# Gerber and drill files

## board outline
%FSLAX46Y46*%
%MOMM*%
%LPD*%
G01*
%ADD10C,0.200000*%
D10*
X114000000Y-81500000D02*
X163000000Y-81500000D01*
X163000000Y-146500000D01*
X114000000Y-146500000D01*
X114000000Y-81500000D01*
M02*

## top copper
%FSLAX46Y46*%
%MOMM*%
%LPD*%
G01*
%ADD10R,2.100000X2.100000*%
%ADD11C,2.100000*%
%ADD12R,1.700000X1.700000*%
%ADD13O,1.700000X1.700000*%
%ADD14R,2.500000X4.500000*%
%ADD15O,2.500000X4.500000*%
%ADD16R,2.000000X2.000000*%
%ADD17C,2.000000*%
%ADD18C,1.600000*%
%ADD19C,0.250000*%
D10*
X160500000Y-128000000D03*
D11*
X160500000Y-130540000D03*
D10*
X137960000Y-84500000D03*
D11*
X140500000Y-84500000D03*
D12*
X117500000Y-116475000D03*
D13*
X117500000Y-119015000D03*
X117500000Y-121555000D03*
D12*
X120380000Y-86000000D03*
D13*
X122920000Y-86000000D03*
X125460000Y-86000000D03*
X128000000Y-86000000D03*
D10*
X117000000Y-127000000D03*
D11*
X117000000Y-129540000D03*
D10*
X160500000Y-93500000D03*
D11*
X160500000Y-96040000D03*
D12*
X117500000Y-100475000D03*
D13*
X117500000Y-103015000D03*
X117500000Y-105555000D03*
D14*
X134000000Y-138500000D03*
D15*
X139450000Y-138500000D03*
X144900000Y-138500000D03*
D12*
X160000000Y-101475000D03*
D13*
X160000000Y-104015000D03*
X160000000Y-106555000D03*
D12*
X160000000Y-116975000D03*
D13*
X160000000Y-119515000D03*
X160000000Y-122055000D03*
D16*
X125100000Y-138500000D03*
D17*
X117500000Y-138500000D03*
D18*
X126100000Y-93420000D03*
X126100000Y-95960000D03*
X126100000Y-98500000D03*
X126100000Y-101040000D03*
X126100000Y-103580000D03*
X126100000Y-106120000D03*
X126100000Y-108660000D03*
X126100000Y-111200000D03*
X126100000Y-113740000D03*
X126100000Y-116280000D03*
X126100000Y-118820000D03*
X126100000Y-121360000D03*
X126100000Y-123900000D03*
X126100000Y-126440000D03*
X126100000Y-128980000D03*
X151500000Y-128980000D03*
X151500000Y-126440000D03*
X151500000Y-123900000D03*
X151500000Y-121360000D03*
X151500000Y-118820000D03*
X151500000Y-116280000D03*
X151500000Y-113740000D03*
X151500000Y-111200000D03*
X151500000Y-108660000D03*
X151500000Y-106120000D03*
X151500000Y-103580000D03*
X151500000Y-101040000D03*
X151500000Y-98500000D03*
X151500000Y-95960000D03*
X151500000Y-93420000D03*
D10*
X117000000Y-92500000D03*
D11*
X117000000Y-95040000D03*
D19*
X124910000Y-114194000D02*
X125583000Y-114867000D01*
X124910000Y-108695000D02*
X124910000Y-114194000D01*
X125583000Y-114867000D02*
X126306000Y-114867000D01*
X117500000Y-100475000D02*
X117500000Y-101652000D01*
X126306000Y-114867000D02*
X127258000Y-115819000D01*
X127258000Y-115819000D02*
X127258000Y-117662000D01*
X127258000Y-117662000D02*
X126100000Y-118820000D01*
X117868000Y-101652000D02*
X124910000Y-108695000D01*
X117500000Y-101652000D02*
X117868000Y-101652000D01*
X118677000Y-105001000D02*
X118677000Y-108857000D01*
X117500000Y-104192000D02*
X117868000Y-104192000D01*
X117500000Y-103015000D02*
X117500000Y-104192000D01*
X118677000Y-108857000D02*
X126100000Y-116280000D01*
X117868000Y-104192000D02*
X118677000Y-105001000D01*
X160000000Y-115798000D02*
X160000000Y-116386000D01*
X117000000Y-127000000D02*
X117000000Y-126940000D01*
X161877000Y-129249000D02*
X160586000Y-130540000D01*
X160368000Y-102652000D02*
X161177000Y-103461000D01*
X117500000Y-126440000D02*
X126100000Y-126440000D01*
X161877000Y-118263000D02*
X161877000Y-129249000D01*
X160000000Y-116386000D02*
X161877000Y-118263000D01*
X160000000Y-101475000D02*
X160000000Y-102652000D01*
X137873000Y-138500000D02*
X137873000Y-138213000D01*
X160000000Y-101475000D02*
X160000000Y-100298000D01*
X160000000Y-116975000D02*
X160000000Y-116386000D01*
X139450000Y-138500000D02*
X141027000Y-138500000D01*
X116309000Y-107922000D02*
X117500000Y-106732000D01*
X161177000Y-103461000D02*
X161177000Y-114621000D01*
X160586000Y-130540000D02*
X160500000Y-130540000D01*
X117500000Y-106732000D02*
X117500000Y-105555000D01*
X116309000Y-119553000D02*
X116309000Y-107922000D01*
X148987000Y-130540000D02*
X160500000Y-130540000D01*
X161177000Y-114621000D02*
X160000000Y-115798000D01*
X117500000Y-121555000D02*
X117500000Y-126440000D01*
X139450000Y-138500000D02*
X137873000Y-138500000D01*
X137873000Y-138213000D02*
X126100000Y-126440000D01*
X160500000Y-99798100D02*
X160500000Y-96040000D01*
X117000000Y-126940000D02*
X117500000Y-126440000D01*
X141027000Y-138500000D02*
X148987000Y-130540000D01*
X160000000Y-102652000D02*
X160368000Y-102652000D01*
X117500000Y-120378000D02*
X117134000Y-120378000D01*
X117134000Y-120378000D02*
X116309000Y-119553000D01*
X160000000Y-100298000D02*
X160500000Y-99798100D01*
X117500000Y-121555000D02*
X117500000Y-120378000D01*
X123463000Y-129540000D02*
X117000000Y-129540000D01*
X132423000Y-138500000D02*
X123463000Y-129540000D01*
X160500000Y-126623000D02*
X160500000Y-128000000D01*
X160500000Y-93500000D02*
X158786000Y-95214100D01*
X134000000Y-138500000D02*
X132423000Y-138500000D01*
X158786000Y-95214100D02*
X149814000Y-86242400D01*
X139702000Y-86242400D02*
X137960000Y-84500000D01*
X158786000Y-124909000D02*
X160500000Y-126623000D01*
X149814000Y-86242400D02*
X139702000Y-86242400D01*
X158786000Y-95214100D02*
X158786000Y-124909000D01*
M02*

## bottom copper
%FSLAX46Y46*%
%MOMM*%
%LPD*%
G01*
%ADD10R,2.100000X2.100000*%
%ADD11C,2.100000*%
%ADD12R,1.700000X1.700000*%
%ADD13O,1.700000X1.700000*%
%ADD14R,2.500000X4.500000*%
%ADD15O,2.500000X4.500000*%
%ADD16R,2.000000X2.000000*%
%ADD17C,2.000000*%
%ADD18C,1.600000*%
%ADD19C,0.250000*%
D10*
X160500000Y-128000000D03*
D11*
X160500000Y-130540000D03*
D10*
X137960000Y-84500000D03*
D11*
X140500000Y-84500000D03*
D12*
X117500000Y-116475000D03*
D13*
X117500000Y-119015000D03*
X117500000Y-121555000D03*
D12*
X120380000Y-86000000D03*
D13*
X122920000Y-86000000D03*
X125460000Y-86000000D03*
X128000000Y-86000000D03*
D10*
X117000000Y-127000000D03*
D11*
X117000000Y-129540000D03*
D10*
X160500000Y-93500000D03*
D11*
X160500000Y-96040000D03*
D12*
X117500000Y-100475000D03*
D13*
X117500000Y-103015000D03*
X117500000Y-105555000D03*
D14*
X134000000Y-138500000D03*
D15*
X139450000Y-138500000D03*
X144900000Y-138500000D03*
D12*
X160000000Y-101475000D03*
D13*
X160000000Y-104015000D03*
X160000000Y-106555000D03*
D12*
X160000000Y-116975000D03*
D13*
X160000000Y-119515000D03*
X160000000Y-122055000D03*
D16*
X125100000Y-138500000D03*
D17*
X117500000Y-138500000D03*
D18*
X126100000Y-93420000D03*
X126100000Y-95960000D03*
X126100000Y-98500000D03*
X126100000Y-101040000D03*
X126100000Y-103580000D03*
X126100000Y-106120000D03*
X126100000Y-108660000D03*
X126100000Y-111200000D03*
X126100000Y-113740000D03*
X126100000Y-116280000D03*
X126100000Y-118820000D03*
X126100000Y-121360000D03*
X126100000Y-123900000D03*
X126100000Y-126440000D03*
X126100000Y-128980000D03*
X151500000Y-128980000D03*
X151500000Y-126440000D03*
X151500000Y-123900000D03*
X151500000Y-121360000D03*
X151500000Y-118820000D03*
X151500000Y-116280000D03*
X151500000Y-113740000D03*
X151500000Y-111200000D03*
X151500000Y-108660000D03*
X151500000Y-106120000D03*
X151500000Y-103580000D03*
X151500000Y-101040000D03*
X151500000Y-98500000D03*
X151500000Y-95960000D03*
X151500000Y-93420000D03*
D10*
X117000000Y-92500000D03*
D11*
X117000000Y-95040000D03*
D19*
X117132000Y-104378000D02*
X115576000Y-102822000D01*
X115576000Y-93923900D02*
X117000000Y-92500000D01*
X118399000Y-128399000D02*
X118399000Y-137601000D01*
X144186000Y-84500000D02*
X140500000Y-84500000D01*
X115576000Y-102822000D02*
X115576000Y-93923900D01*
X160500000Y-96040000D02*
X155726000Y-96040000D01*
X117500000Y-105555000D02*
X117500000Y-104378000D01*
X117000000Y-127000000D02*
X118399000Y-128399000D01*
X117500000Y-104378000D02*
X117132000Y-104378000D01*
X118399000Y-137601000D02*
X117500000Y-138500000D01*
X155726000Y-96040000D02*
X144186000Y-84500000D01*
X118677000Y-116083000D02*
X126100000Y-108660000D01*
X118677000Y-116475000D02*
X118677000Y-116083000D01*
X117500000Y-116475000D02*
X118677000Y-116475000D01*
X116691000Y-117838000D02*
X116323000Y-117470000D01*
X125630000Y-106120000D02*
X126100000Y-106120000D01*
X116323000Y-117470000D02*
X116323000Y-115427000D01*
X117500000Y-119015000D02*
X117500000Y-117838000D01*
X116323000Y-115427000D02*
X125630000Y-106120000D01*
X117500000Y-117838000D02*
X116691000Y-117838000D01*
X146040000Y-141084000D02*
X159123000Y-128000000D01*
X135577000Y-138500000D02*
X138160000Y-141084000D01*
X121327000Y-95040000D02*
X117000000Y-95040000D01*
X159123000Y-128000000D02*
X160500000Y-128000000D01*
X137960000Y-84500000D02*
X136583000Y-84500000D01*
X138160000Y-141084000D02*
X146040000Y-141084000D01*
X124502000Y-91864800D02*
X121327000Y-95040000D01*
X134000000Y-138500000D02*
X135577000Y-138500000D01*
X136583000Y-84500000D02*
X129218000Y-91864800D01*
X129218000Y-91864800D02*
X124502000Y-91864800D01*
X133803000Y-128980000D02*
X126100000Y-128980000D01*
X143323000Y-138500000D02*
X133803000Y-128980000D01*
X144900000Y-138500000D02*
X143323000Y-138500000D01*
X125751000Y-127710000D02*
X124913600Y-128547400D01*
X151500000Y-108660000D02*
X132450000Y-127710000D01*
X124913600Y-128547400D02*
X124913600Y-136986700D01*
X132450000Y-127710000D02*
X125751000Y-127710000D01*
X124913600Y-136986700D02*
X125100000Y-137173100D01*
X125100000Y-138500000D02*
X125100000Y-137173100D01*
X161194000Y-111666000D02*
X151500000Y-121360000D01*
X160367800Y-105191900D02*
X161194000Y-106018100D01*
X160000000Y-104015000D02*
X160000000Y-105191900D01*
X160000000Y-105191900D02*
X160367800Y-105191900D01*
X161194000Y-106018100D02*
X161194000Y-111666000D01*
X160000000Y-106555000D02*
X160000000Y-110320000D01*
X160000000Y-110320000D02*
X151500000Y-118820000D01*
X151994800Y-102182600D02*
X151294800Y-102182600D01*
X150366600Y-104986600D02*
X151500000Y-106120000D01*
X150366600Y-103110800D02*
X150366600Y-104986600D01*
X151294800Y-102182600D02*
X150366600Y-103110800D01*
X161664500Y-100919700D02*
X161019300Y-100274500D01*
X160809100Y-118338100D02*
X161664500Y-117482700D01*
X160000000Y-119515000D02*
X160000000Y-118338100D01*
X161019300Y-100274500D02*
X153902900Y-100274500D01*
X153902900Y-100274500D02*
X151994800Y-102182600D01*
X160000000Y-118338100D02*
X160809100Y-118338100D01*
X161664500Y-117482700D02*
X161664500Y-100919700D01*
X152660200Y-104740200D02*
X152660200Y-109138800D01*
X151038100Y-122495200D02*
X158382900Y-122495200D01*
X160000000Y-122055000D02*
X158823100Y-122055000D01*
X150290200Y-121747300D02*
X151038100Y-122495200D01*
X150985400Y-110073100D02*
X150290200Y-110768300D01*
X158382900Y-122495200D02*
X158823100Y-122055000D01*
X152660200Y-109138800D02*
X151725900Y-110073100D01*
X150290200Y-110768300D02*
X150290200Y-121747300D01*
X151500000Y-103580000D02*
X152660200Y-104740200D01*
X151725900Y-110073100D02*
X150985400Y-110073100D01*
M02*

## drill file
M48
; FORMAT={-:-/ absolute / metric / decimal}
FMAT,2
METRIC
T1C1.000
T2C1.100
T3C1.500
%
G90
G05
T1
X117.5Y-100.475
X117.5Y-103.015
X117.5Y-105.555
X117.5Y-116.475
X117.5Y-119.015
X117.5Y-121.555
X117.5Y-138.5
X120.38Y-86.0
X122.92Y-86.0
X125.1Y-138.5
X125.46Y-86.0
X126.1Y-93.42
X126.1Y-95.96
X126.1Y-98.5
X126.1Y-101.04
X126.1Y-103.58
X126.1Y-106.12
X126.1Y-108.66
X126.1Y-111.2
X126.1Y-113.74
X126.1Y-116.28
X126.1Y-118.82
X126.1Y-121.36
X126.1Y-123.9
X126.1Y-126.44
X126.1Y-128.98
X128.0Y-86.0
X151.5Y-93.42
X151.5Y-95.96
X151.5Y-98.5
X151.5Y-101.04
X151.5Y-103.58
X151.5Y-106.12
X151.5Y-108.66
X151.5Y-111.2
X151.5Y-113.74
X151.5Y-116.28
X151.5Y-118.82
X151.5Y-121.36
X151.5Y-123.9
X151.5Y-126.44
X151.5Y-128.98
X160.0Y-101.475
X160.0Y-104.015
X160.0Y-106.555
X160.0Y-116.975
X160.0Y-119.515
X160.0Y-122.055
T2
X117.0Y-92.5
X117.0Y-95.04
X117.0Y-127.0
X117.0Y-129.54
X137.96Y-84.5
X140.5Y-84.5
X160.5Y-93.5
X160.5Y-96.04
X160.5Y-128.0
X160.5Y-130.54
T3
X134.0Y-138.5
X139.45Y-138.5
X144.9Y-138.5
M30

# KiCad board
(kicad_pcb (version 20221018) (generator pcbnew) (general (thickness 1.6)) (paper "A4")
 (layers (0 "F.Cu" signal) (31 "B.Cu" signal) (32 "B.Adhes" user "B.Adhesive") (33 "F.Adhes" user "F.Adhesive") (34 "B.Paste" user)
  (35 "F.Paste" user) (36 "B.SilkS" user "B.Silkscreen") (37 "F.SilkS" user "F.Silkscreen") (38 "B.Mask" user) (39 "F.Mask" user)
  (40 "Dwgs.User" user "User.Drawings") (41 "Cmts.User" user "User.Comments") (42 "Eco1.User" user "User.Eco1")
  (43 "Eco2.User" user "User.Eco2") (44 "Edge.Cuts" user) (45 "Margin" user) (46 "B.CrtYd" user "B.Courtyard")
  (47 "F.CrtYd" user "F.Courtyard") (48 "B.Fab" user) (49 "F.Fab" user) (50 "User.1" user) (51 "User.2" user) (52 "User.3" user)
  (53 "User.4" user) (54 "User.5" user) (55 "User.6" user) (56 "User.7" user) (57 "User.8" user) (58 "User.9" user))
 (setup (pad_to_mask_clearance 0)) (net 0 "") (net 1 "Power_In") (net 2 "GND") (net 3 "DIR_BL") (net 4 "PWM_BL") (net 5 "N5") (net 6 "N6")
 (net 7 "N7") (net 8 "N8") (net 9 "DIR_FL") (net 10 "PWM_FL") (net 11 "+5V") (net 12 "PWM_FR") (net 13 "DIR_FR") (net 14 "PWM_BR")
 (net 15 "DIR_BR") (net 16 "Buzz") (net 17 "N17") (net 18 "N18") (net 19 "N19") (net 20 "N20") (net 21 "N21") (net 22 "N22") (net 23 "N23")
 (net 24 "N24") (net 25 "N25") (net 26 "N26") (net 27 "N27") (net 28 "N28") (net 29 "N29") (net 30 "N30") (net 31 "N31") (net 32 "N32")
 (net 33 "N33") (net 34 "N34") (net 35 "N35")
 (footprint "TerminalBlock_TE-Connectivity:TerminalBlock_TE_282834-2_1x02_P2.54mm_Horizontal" (layer "F.Cu") (at 160.5 128 -90)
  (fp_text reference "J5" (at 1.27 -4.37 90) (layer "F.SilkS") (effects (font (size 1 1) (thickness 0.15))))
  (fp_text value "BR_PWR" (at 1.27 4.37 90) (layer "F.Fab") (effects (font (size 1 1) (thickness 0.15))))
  (pad "1" thru_hole rect (at 0 0 270) (size 2.1 2.1) (drill 1.1) (layers "*.Cu" "*.Mask") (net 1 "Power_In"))
  (pad "2" thru_hole circle (at 2.54 0 270) (size 2.1 2.1) (drill 1.1) (layers "*.Cu" "*.Mask") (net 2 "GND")))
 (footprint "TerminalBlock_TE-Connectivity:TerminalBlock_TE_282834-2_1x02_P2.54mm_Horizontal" (layer "F.Cu") (at 137.96 84.5)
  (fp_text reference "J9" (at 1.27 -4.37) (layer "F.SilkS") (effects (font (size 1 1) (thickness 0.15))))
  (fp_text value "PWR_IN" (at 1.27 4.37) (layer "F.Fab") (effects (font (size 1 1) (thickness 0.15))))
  (pad "1" thru_hole rect (at 0 0) (size 2.1 2.1) (drill 1.1) (layers "*.Cu" "*.Mask") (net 1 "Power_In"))
  (pad "2" thru_hole circle (at 2.54 0) (size 2.1 2.1) (drill 1.1) (layers "*.Cu" "*.Mask") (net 2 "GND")))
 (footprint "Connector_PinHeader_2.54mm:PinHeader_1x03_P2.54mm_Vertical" (layer "F.Cu") (at 117.5 116.475)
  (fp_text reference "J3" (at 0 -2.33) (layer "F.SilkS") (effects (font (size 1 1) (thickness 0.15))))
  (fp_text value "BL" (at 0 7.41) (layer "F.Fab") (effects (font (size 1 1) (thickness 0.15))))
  (pad "1" thru_hole rect (at 0 0) (size 1.7 1.7) (drill 1) (layers "*.Cu" "*.Mask") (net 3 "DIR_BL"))
  (pad "2" thru_hole oval (at 0 2.54) (size 1.7 1.7) (drill 1) (layers "*.Cu" "*.Mask") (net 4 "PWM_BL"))
  (pad "3" thru_hole oval (at 0 5.08) (size 1.7 1.7) (drill 1) (layers "*.Cu" "*.Mask") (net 2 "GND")))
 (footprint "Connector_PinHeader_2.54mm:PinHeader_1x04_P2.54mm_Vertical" (layer "F.Cu") (at 120.38 86 90)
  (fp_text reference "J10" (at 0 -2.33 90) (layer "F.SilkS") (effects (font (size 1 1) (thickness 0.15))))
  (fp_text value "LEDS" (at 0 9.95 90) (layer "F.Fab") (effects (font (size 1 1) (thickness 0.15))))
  (pad "1" thru_hole rect (at 0 0 90) (size 1.7 1.7) (drill 1) (layers "*.Cu" "*.Mask") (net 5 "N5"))
  (pad "2" thru_hole oval (at 0 2.54 90) (size 1.7 1.7) (drill 1) (layers "*.Cu" "*.Mask") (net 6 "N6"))
  (pad "3" thru_hole oval (at 0 5.08 90) (size 1.7 1.7) (drill 1) (layers "*.Cu" "*.Mask") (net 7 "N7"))
  (pad "4" thru_hole oval (at 0 7.62 90) (size 1.7 1.7) (drill 1) (layers "*.Cu" "*.Mask") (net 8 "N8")))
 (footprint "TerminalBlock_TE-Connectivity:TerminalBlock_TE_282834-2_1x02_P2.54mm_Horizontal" (layer "F.Cu") (at 117 127 -90)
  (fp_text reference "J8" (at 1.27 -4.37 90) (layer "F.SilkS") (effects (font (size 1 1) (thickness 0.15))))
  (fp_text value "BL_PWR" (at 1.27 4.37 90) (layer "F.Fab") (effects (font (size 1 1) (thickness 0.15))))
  (pad "1" thru_hole rect (at 0 0 270) (size 2.1 2.1) (drill 1.1) (layers "*.Cu" "*.Mask") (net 2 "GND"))
  (pad "2" thru_hole circle (at 2.54 0 270) (size 2.1 2.1) (drill 1.1) (layers "*.Cu" "*.Mask") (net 1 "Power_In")))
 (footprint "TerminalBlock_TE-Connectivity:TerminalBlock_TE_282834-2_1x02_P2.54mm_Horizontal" (layer "F.Cu") (at 160.5 93.5 -90)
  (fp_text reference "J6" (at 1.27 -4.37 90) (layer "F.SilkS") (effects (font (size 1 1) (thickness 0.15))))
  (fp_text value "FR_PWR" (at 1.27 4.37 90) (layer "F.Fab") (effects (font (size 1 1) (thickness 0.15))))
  (pad "1" thru_hole rect (at 0 0 270) (size 2.1 2.1) (drill 1.1) (layers "*.Cu" "*.Mask") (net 1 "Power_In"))
  (pad "2" thru_hole circle (at 2.54 0 270) (size 2.1 2.1) (drill 1.1) (layers "*.Cu" "*.Mask") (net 2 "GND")))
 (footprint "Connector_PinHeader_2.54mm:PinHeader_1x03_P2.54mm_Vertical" (layer "F.Cu") (at 117.5 100.475)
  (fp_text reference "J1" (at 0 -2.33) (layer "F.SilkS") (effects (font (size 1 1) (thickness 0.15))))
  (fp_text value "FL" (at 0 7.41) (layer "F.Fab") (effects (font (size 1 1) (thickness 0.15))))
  (pad "1" thru_hole rect (at 0 0) (size 1.7 1.7) (drill 1) (layers "*.Cu" "*.Mask") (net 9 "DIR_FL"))
  (pad "2" thru_hole oval (at 0 2.54) (size 1.7 1.7) (drill 1) (layers "*.Cu" "*.Mask") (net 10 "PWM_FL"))
  (pad "3" thru_hole oval (at 0 5.08) (size 1.7 1.7) (drill 1) (layers "*.Cu" "*.Mask") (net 2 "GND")))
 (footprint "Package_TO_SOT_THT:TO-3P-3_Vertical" (layer "F.Cu") (at 134 138.5)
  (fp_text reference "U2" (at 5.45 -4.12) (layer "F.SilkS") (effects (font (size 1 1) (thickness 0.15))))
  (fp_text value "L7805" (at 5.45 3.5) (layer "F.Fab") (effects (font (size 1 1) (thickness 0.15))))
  (pad "1" thru_hole rect (at 0 0) (size 2.5 4.5) (drill 1.5) (layers "*.Cu" "*.Mask") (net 1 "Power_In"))
  (pad "2" thru_hole oval (at 5.45 0) (size 2.5 4.5) (drill 1.5) (layers "*.Cu" "*.Mask") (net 2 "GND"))
  (pad "3" thru_hole oval (at 10.9 0) (size 2.5 4.5) (drill 1.5) (layers "*.Cu" "*.Mask") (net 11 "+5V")))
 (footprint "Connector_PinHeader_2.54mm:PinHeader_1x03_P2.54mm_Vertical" (layer "F.Cu") (at 160 101.475)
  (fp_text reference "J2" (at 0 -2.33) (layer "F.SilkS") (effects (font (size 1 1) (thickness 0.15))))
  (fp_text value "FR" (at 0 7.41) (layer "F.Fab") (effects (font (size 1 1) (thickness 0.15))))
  (pad "1" thru_hole rect (at 0 0) (size 1.7 1.7) (drill 1) (layers "*.Cu" "*.Mask") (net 2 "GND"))
  (pad "2" thru_hole oval (at 0 2.54) (size 1.7 1.7) (drill 1) (layers "*.Cu" "*.Mask") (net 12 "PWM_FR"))
  (pad "3" thru_hole oval (at 0 5.08) (size 1.7 1.7) (drill 1) (layers "*.Cu" "*.Mask") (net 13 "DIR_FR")))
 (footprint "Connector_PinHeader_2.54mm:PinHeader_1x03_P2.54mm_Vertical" (layer "F.Cu") (at 160 116.975)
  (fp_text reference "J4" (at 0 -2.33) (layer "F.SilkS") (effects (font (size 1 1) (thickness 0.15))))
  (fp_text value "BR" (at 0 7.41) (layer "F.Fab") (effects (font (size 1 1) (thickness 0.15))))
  (pad "1" thru_hole rect (at 0 0) (size 1.7 1.7) (drill 1) (layers "*.Cu" "*.Mask") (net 2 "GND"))
  (pad "2" thru_hole oval (at 0 2.54) (size 1.7 1.7) (drill 1) (layers "*.Cu" "*.Mask") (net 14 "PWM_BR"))
  (pad "3" thru_hole oval (at 0 5.08) (size 1.7 1.7) (drill 1) (layers "*.Cu" "*.Mask") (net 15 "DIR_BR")))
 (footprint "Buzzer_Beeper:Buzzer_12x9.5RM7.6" (layer "F.Cu") (at 125.1 138.5 180)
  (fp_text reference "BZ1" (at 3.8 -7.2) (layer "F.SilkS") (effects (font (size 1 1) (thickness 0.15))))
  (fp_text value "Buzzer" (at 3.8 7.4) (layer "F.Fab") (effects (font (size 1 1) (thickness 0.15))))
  (pad "1" thru_hole rect (at 0 0 180) (size 2 2) (drill 1) (layers "*.Cu" "*.Mask") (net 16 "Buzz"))
  (pad "2" thru_hole circle (at 7.6 0 180) (size 2 2) (drill 1) (layers "*.Cu" "*.Mask") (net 2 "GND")))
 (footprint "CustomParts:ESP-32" (layer "F.Cu") (at 138.8 111.2)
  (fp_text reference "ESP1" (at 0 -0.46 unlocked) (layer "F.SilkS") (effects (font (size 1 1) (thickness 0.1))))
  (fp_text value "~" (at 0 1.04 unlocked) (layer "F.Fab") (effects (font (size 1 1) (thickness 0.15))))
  (pad "1" thru_hole circle (at -12.7 -17.78) (size 1.6 1.6) (drill 1) (layers "*.Cu" "*.Mask") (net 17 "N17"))
  (pad "2" thru_hole circle (at -12.7 -15.24) (size 1.6 1.6) (drill 1) (layers "*.Cu" "*.Mask") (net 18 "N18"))
  (pad "3" thru_hole circle (at -12.7 -12.7) (size 1.6 1.6) (drill 1) (layers "*.Cu" "*.Mask") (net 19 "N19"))
  (pad "4" thru_hole circle (at -12.7 -10.16) (size 1.6 1.6) (drill 1) (layers "*.Cu" "*.Mask") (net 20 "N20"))
  (pad "5" thru_hole circle (at -12.7 -7.62) (size 1.6 1.6) (drill 1) (layers "*.Cu" "*.Mask") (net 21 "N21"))
  (pad "6" thru_hole circle (at -12.7 -5.08) (size 1.6 1.6) (drill 1) (layers "*.Cu" "*.Mask") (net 4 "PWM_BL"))
  (pad "7" thru_hole circle (at -12.7 -2.54) (size 1.6 1.6) (drill 1) (layers "*.Cu" "*.Mask") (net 3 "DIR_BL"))
  (pad "8" thru_hole circle (at -12.7 0) (size 1.6 1.6) (drill 1) (layers "*.Cu" "*.Mask") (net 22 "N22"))
  (pad "9" thru_hole circle (at -12.7 2.54) (size 1.6 1.6) (drill 1) (layers "*.Cu" "*.Mask") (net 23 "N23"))
  (pad "10" thru_hole circle (at -12.7 5.08) (size 1.6 1.6) (drill 1) (layers "*.Cu" "*.Mask") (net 10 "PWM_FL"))
  (pad "11" thru_hole circle (at -12.7 7.62) (size 1.6 1.6) (drill 1) (layers "*.Cu" "*.Mask") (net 9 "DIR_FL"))
  (pad "12" thru_hole circle (at -12.7 10.16) (size 1.6 1.6) (drill 1) (layers "*.Cu" "*.Mask") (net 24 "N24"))
  (pad "13" thru_hole circle (at -12.7 12.7) (size 1.6 1.6) (drill 1) (layers "*.Cu" "*.Mask") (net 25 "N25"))
  (pad "14" thru_hole circle (at -12.7 15.24) (size 1.6 1.6) (drill 1) (layers "*.Cu" "*.Mask") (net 2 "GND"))
  (pad "15" thru_hole circle (at -12.7 17.78) (size 1.6 1.6) (drill 1) (layers "*.Cu" "*.Mask") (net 11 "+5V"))
  (pad "16" thru_hole circle (at 12.7 17.78) (size 1.6 1.6) (drill 1) (layers "*.Cu" "*.Mask") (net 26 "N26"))
  (pad "17" thru_hole circle (at 12.7 15.24) (size 1.6 1.6) (drill 1) (layers "*.Cu" "*.Mask") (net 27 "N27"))
  (pad "18" thru_hole circle (at 12.7 12.7) (size 1.6 1.6) (drill 1) (layers "*.Cu" "*.Mask") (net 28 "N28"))
  (pad "19" thru_hole circle (at 12.7 10.16) (size 1.6 1.6) (drill 1) (layers "*.Cu" "*.Mask") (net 12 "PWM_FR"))
  (pad "20" thru_hole circle (at 12.7 7.62) (size 1.6 1.6) (drill 1) (layers "*.Cu" "*.Mask") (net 13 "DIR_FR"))
  (pad "21" thru_hole circle (at 12.7 5.08) (size 1.6 1.6) (drill 1) (layers "*.Cu" "*.Mask") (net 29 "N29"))
  (pad "22" thru_hole circle (at 12.7 2.54) (size 1.6 1.6) (drill 1) (layers "*.Cu" "*.Mask") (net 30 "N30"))
  (pad "23" thru_hole circle (at 12.7 0) (size 1.6 1.6) (drill 1) (layers "*.Cu" "*.Mask") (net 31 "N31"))
  (pad "24" thru_hole circle (at 12.7 -2.54) (size 1.6 1.6) (drill 1) (layers "*.Cu" "*.Mask") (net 16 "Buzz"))
  (pad "25" thru_hole circle (at 12.7 -5.08) (size 1.6 1.6) (drill 1) (layers "*.Cu" "*.Mask") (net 14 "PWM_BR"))
  (pad "26" thru_hole circle (at 12.7 -7.62) (size 1.6 1.6) (drill 1) (layers "*.Cu" "*.Mask") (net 15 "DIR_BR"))
  (pad "27" thru_hole circle (at 12.7 -10.16) (size 1.6 1.6) (drill 1) (layers "*.Cu" "*.Mask") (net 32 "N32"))
  (pad "28" thru_hole circle (at 12.7 -12.7) (size 1.6 1.6) (drill 1) (layers "*.Cu" "*.Mask") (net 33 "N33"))
  (pad "29" thru_hole circle (at 12.7 -15.24) (size 1.6 1.6) (drill 1) (layers "*.Cu" "*.Mask") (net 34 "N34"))
  (pad "30" thru_hole circle (at 12.7 -17.78) (size 1.6 1.6) (drill 1) (layers "*.Cu" "*.Mask") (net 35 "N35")))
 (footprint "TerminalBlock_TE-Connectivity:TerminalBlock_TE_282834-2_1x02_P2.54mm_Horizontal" (layer "F.Cu") (at 117 92.5 -90)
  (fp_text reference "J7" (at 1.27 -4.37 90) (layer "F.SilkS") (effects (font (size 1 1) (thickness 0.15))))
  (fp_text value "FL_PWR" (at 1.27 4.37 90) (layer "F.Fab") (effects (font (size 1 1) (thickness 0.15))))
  (pad "1" thru_hole rect (at 0 0 270) (size 2.1 2.1) (drill 1.1) (layers "*.Cu" "*.Mask") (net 2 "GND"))
  (pad "2" thru_hole circle (at 2.54 0 270) (size 2.1 2.1) (drill 1.1) (layers "*.Cu" "*.Mask") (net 1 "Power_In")))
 (gr_rect (start 114 81.5) (end 163 146.5) (stroke (width 0.2) (type default)) (fill none) (layer "Edge.Cuts"))
 (segment (start 124.91 114.194) (end 125.583 114.867) (width 0.25) (layer "F.Cu") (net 9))
 (segment (start 124.91 108.695) (end 124.91 114.194) (width 0.25) (layer "F.Cu") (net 9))
 (segment (start 125.583 114.867) (end 126.306 114.867) (width 0.25) (layer "F.Cu") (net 9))
 (segment (start 117.5 100.475) (end 117.5 101.652) (width 0.25) (layer "F.Cu") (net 9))
 (segment (start 126.306 114.867) (end 127.258 115.819) (width 0.25) (layer "F.Cu") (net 9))
 (segment (start 127.258 115.819) (end 127.258 117.662) (width 0.25) (layer "F.Cu") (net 9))
 (segment (start 127.258 117.662) (end 126.1 118.82) (width 0.25) (layer "F.Cu") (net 9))
 (segment (start 117.868 101.652) (end 124.91 108.695) (width 0.25) (layer "F.Cu") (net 9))
 (segment (start 117.5 101.652) (end 117.868 101.652) (width 0.25) (layer "F.Cu") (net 9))
 (segment (start 118.677 105.001) (end 118.677 108.857) (width 0.25) (layer "F.Cu") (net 10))
 (segment (start 117.5 104.192) (end 117.868 104.192) (width 0.25) (layer "F.Cu") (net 10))
 (segment (start 117.5 103.015) (end 117.5 104.192) (width 0.25) (layer "F.Cu") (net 10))
 (segment (start 118.677 108.857) (end 126.1 116.28) (width 0.25) (layer "F.Cu") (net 10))
 (segment (start 117.868 104.192) (end 118.677 105.001) (width 0.25) (layer "F.Cu") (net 10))
 (segment (start 160 115.798) (end 160 116.386) (width 0.25) (layer "F.Cu") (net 2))
 (segment (start 117 127) (end 117 126.94) (width 0.25) (layer "F.Cu") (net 2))
 (segment (start 161.877 129.249) (end 160.586 130.54) (width 0.25) (layer "F.Cu") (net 2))
 (segment (start 160.368 102.652) (end 161.177 103.461) (width 0.25) (layer "F.Cu") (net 2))
 (segment (start 117.5 126.44) (end 126.1 126.44) (width 0.25) (layer "F.Cu") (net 2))
 (segment (start 161.877 118.263) (end 161.877 129.249) (width 0.25) (layer "F.Cu") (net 2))
 (segment (start 160 116.386) (end 161.877 118.263) (width 0.25) (layer "F.Cu") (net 2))
 (segment (start 160 101.475) (end 160 102.652) (width 0.25) (layer "F.Cu") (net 2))
 (segment (start 137.873 138.5) (end 137.873 138.213) (width 0.25) (layer "F.Cu") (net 2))
 (segment (start 160 101.475) (end 160 100.298) (width 0.25) (layer "F.Cu") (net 2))
 (segment (start 160 116.975) (end 160 116.386) (width 0.25) (layer "F.Cu") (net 2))
 (segment (start 139.45 138.5) (end 141.027 138.5) (width 0.25) (layer "F.Cu") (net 2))
 (segment (start 116.309 107.922) (end 117.5 106.732) (width 0.25) (layer "F.Cu") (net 2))
 (segment (start 161.177 103.461) (end 161.177 114.621) (width 0.25) (layer "F.Cu") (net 2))
 (segment (start 160.586 130.54) (end 160.5 130.54) (width 0.25) (layer "F.Cu") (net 2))
 (segment (start 117.5 106.732) (end 117.5 105.555) (width 0.25) (layer "F.Cu") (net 2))
 (segment (start 116.309 119.553) (end 116.309 107.922) (width 0.25) (layer "F.Cu") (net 2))
 (segment (start 148.987 130.54) (end 160.5 130.54) (width 0.25) (layer "F.Cu") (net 2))
 (segment (start 161.177 114.621) (end 160 115.798) (width 0.25) (layer "F.Cu") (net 2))
 (segment (start 117.5 121.555) (end 117.5 126.44) (width 0.25) (layer "F.Cu") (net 2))
 (segment (start 139.45 138.5) (end 137.873 138.5) (width 0.25) (layer "F.Cu") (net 2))
 (segment (start 137.873 138.213) (end 126.1 126.44) (width 0.25) (layer "F.Cu") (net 2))
 (segment (start 160.5 99.7981) (end 160.5 96.04) (width 0.25) (layer "F.Cu") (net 2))
 (segment (start 117 126.94) (end 117.5 126.44) (width 0.25) (layer "F.Cu") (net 2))
 (segment (start 141.027 138.5) (end 148.987 130.54) (width 0.25) (layer "F.Cu") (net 2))
 (segment (start 160 102.652) (end 160.368 102.652) (width 0.25) (layer "F.Cu") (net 2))
 (segment (start 117.5 120.378) (end 117.134 120.378) (width 0.25) (layer "F.Cu") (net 2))
 (segment (start 117.134 120.378) (end 116.309 119.553) (width 0.25) (layer "F.Cu") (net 2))
 (segment (start 160 100.298) (end 160.5 99.7981) (width 0.25) (layer "F.Cu") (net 2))
 (segment (start 117.5 121.555) (end 117.5 120.378) (width 0.25) (layer "F.Cu") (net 2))
 (segment (start 117.132 104.378) (end 115.576 102.822) (width 0.25) (layer "B.Cu") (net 2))
 (segment (start 115.576 93.9239) (end 117 92.5) (width 0.25) (layer "B.Cu") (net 2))
 (segment (start 118.399 128.399) (end 118.399 137.601) (width 0.25) (layer "B.Cu") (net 2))
 (segment (start 144.186 84.5) (end 140.5 84.5) (width 0.25) (layer "B.Cu") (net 2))
 (segment (start 115.576 102.822) (end 115.576 93.9239) (width 0.25) (layer "B.Cu") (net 2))
 (segment (start 160.5 96.04) (end 155.726 96.04) (width 0.25) (layer "B.Cu") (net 2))
 (segment (start 117.5 105.555) (end 117.5 104.378) (width 0.25) (layer "B.Cu") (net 2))
 (segment (start 117 127) (end 118.399 128.399) (width 0.25) (layer "B.Cu") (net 2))
 (segment (start 117.5 104.378) (end 117.132 104.378) (width 0.25) (layer "B.Cu") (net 2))
 (segment (start 118.399 137.601) (end 117.5 138.5) (width 0.25) (layer "B.Cu") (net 2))
 (segment (start 155.726 96.04) (end 144.186 84.5) (width 0.25) (layer "B.Cu") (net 2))
 (segment (start 118.677 116.083) (end 126.1 108.66) (width 0.25) (layer "B.Cu") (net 3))
 (segment (start 118.677 116.475) (end 118.677 116.083) (width 0.25) (layer "B.Cu") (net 3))
 (segment (start 117.5 116.475) (end 118.677 116.475) (width 0.25) (layer "B.Cu") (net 3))
 (segment (start 116.691 117.838) (end 116.323 117.47) (width 0.25) (layer "B.Cu") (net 4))
 (segment (start 125.63 106.12) (end 126.1 106.12) (width 0.25) (layer "B.Cu") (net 4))
 (segment (start 116.323 117.47) (end 116.323 115.427) (width 0.25) (layer "B.Cu") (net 4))
 (segment (start 117.5 119.015) (end 117.5 117.838) (width 0.25) (layer "B.Cu") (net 4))
 (segment (start 116.323 115.427) (end 125.63 106.12) (width 0.25) (layer "B.Cu") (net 4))
 (segment (start 117.5 117.838) (end 116.691 117.838) (width 0.25) (layer "B.Cu") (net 4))
 (segment (start 123.463 129.54) (end 117 129.54) (width 0.25) (layer "F.Cu") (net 1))
 (segment (start 132.423 138.5) (end 123.463 129.54) (width 0.25) (layer "F.Cu") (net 1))
 (segment (start 160.5 126.623) (end 160.5 128) (width 0.25) (layer "F.Cu") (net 1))
 (segment (start 160.5 93.5) (end 158.786 95.2141) (width 0.25) (layer "F.Cu") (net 1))
 (segment (start 134 138.5) (end 132.423 138.5) (width 0.25) (layer "F.Cu") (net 1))
 (segment (start 158.786 95.2141) (end 149.814 86.2424) (width 0.25) (layer "F.Cu") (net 1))
 (segment (start 139.702 86.2424) (end 137.96 84.5) (width 0.25) (layer "F.Cu") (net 1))
 (segment (start 158.786 124.909) (end 160.5 126.623) (width 0.25) (layer "F.Cu") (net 1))
 (segment (start 149.814 86.2424) (end 139.702 86.2424) (width 0.25) (layer "F.Cu") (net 1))
 (segment (start 158.786 95.2141) (end 158.786 124.909) (width 0.25) (layer "F.Cu") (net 1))
 (segment (start 146.04 141.084) (end 159.123 128) (width 0.25) (layer "B.Cu") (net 1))
 (segment (start 135.577 138.5) (end 138.16 141.084) (width 0.25) (layer "B.Cu") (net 1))
 (segment (start 121.327 95.04) (end 117 95.04) (width 0.25) (layer "B.Cu") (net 1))
 (segment (start 159.123 128) (end 160.5 128) (width 0.25) (layer "B.Cu") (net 1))
 (segment (start 137.96 84.5) (end 136.583 84.5) (width 0.25) (layer "B.Cu") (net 1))
 (segment (start 138.16 141.084) (end 146.04 141.084) (width 0.25) (layer "B.Cu") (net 1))
 (segment (start 124.502 91.8648) (end 121.327 95.04) (width 0.25) (layer "B.Cu") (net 1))
 (segment (start 134 138.5) (end 135.577 138.5) (width 0.25) (layer "B.Cu") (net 1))
 (segment (start 136.583 84.5) (end 129.218 91.8648) (width 0.25) (layer "B.Cu") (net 1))
 (segment (start 129.218 91.8648) (end 124.502 91.8648) (width 0.25) (layer "B.Cu") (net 1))
 (segment (start 133.803 128.98) (end 126.1 128.98) (width 0.25) (layer "B.Cu") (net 11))
 (segment (start 143.323 138.5) (end 133.803 128.98) (width 0.25) (layer "B.Cu") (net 11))
 (segment (start 144.9 138.5) (end 143.323 138.5) (width 0.25) (layer "B.Cu") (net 11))
 (segment (start 125.751 127.71) (end 124.9136 128.5474) (width 0.25) (layer "B.Cu") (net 16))
 (segment (start 151.5 108.66) (end 132.45 127.71) (width 0.25) (layer "B.Cu") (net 16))
 (segment (start 124.9136 128.5474) (end 124.9136 136.9867) (width 0.25) (layer "B.Cu") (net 16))
 (segment (start 132.45 127.71) (end 125.751 127.71) (width 0.25) (layer "B.Cu") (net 16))
 (segment (start 124.9136 136.9867) (end 125.1 137.1731) (width 0.25) (layer "B.Cu") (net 16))
 (segment (start 125.1 138.5) (end 125.1 137.1731) (width 0.25) (layer "B.Cu") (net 16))
 (segment (start 161.194 111.666) (end 151.5 121.36) (width 0.25) (layer "B.Cu") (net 12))
 (segment (start 160.3678 105.1919) (end 161.194 106.0181) (width 0.25) (layer "B.Cu") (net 12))
 (segment (start 160 104.015) (end 160 105.1919) (width 0.25) (layer "B.Cu") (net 12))
 (segment (start 160 105.1919) (end 160.3678 105.1919) (width 0.25) (layer "B.Cu") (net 12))
 (segment (start 161.194 106.0181) (end 161.194 111.666) (width 0.25) (layer "B.Cu") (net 12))
 (segment (start 160 106.555) (end 160 110.32) (width 0.25) (layer "B.Cu") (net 13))
 (segment (start 160 110.32) (end 151.5 118.82) (width 0.25) (layer "B.Cu") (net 13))
 (segment (start 151.9948 102.1826) (end 151.2948 102.1826) (width 0.25) (layer "B.Cu") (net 14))
 (segment (start 150.3666 104.9866) (end 151.5 106.12) (width 0.25) (layer "B.Cu") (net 14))
 (segment (start 150.3666 103.1108) (end 150.3666 104.9866) (width 0.25) (layer "B.Cu") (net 14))
 (segment (start 151.2948 102.1826) (end 150.3666 103.1108) (width 0.25) (layer "B.Cu") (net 14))
 (segment (start 161.6645 100.9197) (end 161.0193 100.2745) (width 0.25) (layer "B.Cu") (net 14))
 (segment (start 160.8091 118.3381) (end 161.6645 117.4827) (width 0.25) (layer "B.Cu") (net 14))
 (segment (start 160 119.515) (end 160 118.3381) (width 0.25) (layer "B.Cu") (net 14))
 (segment (start 161.0193 100.2745) (end 153.9029 100.2745) (width 0.25) (layer "B.Cu") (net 14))
 (segment (start 153.9029 100.2745) (end 151.9948 102.1826) (width 0.25) (layer "B.Cu") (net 14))
 (segment (start 160 118.3381) (end 160.8091 118.3381) (width 0.25) (layer "B.Cu") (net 14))
 (segment (start 161.6645 117.4827) (end 161.6645 100.9197) (width 0.25) (layer "B.Cu") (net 14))
 (segment (start 152.6602 104.7402) (end 152.6602 109.1388) (width 0.25) (layer "B.Cu") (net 15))
 (segment (start 151.0381 122.4952) (end 158.3829 122.4952) (width 0.25) (layer "B.Cu") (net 15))
 (segment (start 160 122.055) (end 158.8231 122.055) (width 0.25) (layer "B.Cu") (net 15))
 (segment (start 150.2902 121.7473) (end 151.0381 122.4952) (width 0.25) (layer "B.Cu") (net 15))
 (segment (start 150.9854 110.0731) (end 150.2902 110.7683) (width 0.25) (layer "B.Cu") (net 15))
 (segment (start 158.3829 122.4952) (end 158.8231 122.055) (width 0.25) (layer "B.Cu") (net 15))
 (segment (start 152.6602 109.1388) (end 151.7259 110.0731) (width 0.25) (layer "B.Cu") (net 15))
 (segment (start 150.2902 110.7683) (end 150.2902 121.7473) (width 0.25) (layer "B.Cu") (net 15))
 (segment (start 151.5 103.58) (end 152.6602 104.7402) (width 0.25) (layer "B.Cu") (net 15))
 (segment (start 151.7259 110.0731) (end 150.9854 110.0731) (width 0.25) (layer "B.Cu") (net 15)))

